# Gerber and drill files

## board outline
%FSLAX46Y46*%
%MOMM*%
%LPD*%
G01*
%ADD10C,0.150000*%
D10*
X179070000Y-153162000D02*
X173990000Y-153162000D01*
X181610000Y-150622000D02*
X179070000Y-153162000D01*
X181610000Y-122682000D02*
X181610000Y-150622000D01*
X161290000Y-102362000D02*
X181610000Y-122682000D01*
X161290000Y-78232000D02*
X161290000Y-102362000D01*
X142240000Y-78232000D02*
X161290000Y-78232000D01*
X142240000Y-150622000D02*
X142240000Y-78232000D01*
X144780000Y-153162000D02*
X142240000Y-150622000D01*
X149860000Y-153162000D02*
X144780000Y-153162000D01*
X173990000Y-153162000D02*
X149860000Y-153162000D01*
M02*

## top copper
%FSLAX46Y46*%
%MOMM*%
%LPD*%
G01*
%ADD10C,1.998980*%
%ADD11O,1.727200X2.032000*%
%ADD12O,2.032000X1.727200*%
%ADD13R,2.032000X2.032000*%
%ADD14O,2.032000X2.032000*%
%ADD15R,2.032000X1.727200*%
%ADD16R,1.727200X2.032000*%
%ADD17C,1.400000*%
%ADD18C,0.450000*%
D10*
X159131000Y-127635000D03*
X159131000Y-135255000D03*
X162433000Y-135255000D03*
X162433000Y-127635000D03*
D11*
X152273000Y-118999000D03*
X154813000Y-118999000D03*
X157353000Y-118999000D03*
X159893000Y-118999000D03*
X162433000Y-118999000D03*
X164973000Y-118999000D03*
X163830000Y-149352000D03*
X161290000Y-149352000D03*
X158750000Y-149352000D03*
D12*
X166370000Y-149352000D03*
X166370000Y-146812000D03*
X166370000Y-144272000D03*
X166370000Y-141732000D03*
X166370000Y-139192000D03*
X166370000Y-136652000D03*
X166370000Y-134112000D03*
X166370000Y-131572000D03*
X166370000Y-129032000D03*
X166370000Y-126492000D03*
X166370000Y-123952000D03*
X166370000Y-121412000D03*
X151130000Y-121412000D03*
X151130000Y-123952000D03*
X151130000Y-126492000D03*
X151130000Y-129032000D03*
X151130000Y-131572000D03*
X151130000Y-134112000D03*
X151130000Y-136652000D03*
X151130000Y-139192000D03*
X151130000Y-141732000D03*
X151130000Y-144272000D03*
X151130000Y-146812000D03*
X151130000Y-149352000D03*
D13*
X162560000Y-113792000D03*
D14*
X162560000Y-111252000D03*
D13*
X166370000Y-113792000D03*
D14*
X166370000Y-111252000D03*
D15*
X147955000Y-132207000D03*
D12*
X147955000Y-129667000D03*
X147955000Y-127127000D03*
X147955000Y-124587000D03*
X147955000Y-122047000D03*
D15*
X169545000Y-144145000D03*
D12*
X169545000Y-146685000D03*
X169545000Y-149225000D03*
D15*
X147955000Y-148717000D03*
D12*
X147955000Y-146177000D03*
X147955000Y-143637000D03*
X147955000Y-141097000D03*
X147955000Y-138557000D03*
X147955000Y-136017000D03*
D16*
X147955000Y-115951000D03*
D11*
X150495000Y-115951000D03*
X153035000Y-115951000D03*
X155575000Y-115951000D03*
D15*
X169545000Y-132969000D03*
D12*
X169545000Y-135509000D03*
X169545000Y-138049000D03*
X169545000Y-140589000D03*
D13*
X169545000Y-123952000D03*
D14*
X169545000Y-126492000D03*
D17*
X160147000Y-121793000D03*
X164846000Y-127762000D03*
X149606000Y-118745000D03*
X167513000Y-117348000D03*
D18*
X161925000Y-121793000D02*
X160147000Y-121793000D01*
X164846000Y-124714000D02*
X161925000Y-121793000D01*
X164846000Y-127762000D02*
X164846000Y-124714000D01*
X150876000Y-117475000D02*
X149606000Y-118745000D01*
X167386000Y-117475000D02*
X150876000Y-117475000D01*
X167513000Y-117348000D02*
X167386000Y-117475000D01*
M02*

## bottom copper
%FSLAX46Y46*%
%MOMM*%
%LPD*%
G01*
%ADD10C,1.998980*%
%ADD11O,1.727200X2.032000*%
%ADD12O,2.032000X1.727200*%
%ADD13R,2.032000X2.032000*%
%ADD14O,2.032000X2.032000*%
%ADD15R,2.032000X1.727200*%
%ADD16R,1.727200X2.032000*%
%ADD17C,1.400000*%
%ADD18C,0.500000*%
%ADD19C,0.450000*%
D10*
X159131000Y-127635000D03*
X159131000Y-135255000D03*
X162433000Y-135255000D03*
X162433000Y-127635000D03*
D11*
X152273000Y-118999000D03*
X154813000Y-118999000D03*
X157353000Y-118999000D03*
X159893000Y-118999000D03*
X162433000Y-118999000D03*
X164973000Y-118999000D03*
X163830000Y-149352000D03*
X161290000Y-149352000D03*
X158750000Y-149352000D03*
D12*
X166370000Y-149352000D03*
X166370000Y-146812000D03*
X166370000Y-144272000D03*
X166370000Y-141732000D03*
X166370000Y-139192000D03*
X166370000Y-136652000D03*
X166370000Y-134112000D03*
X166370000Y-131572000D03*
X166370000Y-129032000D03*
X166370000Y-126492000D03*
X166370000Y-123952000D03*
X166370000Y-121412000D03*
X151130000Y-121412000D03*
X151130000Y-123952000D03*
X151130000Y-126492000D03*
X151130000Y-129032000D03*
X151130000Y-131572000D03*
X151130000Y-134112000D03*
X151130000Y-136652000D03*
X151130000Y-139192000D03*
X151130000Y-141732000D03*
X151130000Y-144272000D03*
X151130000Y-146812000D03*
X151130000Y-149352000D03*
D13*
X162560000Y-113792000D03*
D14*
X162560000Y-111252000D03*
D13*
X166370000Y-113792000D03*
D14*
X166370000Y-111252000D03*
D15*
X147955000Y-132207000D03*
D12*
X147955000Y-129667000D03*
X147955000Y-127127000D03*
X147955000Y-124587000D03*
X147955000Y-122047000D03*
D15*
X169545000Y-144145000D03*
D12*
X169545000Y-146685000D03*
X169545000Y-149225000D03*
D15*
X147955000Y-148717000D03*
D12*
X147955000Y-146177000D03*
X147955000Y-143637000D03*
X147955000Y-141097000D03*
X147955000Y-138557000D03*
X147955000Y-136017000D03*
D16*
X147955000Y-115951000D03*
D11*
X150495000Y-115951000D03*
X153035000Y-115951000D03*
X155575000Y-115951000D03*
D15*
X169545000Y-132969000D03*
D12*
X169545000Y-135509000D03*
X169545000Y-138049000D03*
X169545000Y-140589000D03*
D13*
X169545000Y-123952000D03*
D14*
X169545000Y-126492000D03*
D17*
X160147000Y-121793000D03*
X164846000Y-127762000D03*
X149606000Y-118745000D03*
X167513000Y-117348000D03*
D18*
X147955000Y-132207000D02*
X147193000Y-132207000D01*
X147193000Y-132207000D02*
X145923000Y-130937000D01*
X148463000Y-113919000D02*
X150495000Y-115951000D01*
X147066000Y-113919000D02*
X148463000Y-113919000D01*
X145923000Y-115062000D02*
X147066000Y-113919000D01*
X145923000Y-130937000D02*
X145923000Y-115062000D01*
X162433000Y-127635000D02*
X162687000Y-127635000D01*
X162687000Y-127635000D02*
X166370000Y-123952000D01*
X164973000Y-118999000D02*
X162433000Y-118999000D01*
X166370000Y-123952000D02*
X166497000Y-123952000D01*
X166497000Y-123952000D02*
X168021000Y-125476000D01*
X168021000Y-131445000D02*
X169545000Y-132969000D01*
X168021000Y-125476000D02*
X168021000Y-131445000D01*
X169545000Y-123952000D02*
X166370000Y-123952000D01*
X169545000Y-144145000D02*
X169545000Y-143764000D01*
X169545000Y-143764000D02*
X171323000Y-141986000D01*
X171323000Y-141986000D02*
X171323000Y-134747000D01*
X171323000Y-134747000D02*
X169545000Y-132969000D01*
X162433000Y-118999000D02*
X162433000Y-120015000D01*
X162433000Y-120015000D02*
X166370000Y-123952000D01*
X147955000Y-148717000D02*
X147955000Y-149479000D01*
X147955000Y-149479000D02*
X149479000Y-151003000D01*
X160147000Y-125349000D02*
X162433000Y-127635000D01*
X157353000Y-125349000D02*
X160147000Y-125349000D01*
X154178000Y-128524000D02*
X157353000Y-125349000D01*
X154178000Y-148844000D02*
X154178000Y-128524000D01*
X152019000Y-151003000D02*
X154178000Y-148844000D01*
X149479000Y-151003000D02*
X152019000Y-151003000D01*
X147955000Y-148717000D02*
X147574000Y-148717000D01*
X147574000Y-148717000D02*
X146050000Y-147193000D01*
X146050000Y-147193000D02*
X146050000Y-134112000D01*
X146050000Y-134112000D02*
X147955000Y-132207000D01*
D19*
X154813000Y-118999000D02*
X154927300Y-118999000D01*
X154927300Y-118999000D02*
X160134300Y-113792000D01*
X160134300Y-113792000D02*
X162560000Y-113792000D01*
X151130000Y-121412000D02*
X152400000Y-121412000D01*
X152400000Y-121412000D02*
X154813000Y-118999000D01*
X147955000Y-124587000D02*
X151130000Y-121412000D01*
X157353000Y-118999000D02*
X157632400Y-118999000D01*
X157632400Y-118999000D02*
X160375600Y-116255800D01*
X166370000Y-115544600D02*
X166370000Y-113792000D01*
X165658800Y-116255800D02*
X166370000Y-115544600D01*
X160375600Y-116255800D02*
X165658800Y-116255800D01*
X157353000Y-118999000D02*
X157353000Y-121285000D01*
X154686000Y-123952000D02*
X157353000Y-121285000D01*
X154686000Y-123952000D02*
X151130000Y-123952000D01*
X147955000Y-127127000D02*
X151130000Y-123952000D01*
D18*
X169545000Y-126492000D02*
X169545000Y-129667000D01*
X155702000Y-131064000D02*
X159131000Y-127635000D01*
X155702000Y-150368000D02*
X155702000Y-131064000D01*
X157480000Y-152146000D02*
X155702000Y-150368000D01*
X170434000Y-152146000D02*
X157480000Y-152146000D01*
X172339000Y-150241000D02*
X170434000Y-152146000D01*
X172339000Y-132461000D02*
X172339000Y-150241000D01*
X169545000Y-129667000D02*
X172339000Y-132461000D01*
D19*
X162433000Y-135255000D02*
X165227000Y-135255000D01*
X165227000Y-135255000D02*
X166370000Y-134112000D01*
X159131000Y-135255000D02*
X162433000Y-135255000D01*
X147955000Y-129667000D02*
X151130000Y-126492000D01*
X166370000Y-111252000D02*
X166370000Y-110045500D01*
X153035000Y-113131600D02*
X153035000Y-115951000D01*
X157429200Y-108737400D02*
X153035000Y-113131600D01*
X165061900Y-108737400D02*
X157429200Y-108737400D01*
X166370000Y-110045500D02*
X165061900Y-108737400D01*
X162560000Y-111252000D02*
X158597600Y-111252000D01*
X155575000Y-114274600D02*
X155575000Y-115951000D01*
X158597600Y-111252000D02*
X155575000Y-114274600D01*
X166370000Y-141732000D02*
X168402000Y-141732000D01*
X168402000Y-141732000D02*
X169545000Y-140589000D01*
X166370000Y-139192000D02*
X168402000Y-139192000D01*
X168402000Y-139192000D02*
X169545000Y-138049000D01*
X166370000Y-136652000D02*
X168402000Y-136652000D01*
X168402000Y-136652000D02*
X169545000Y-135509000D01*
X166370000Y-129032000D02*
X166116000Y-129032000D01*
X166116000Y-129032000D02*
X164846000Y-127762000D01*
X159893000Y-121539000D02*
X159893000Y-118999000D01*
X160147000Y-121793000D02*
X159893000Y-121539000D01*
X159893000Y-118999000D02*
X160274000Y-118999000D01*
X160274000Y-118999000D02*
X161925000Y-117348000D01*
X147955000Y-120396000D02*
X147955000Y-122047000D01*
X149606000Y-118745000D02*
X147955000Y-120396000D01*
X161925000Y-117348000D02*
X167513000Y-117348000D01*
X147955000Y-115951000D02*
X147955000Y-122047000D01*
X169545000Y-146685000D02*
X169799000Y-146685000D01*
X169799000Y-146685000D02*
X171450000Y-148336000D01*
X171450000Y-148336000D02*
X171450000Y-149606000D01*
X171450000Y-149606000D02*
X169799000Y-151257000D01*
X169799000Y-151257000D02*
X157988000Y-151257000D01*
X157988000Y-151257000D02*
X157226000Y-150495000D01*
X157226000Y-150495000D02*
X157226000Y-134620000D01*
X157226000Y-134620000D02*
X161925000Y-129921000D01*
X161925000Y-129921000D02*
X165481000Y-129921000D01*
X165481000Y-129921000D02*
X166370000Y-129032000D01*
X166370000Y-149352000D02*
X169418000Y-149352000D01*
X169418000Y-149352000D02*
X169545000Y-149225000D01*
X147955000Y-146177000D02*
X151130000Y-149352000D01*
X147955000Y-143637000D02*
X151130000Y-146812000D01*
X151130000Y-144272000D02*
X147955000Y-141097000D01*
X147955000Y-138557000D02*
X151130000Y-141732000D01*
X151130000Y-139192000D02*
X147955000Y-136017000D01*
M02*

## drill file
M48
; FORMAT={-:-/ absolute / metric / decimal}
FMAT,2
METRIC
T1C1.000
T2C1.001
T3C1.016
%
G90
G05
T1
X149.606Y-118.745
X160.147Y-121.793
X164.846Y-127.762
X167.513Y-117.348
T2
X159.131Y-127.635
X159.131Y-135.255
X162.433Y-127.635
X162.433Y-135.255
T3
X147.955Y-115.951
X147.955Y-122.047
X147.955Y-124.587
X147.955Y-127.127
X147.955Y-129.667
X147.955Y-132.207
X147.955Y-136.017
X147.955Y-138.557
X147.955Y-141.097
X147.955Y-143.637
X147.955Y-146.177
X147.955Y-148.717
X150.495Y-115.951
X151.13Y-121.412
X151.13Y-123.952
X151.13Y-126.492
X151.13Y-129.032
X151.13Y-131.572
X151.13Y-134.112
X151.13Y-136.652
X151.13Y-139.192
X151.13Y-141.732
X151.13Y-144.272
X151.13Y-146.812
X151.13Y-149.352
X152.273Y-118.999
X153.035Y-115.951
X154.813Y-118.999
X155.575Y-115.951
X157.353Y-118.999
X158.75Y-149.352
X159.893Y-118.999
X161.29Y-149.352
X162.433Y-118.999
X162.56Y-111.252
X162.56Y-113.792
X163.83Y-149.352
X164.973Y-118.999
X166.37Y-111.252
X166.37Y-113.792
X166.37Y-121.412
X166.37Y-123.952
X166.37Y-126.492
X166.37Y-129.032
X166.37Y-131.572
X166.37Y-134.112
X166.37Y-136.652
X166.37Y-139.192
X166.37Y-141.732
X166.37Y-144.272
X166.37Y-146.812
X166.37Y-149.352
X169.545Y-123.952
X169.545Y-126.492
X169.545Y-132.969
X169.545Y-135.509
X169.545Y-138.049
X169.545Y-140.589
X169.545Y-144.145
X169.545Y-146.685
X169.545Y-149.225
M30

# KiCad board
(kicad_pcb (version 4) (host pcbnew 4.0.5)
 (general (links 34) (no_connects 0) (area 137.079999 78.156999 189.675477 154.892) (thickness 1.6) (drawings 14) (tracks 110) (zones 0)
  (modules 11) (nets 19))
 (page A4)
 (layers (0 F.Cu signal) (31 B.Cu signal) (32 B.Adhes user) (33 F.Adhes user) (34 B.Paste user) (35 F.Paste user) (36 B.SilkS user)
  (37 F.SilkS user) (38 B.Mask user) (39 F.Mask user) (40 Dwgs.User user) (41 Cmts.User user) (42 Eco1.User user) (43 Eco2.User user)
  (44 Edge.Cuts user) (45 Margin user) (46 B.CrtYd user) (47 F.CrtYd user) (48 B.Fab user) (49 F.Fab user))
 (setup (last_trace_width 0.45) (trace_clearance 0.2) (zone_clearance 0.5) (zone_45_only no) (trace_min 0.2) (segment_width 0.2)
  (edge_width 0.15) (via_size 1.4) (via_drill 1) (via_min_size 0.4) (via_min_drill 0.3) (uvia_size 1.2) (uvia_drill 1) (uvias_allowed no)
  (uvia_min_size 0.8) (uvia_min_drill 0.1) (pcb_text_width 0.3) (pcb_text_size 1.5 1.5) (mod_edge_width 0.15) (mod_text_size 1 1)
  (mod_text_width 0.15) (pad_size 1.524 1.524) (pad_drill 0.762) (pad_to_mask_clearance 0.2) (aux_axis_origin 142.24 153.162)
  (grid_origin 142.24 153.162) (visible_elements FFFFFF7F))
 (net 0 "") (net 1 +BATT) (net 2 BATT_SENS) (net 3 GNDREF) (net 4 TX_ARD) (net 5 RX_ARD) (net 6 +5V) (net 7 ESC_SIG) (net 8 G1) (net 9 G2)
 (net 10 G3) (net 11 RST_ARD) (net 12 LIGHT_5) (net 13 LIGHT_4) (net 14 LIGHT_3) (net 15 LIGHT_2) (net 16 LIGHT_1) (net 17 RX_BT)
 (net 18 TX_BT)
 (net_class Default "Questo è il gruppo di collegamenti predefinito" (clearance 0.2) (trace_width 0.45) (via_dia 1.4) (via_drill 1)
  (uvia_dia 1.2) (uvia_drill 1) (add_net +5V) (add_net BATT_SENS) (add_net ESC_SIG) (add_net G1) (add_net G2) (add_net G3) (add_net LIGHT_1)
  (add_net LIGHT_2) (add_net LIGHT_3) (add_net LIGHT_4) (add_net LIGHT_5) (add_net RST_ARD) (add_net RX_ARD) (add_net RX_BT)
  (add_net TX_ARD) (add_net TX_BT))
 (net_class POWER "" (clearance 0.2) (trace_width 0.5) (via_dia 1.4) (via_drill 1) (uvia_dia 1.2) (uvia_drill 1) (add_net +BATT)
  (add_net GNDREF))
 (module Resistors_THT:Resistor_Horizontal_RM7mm (layer F.Cu) (at 159.131 127.635 270)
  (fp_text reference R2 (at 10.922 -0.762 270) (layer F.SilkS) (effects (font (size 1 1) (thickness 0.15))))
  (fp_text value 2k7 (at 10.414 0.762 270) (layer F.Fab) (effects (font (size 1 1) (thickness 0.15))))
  (pad 1 thru_hole circle (at 0 0 270) (size 1.99898 1.99898) (drill 1.00076) (layers *.Cu *.SilkS *.Mask) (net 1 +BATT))
  (pad 2 thru_hole circle (at 7.62 0 270) (size 1.99898 1.99898) (drill 1.00076) (layers *.Cu *.SilkS *.Mask) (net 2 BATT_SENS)))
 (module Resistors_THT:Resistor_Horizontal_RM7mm (layer F.Cu) (at 162.433 135.255 90)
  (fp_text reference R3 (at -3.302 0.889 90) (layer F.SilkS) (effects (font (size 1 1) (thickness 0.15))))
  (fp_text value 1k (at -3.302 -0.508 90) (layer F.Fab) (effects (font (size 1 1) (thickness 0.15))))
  (pad 1 thru_hole circle (at 0 0 90) (size 1.99898 1.99898) (drill 1.00076) (layers *.Cu *.SilkS *.Mask) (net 2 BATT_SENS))
  (pad 2 thru_hole circle (at 7.62 0 90) (size 1.99898 1.99898) (drill 1.00076) (layers *.Cu *.SilkS *.Mask) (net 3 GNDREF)))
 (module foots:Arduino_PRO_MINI (layer F.Cu) (at 158.75 118.872)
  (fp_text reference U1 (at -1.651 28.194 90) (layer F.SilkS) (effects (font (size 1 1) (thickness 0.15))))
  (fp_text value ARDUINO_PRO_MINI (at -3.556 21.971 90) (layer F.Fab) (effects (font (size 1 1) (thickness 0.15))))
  (pad 33 thru_hole oval (at -6.477 0.127 90) (size 2.032 1.7272) (drill 1.016) (layers *.Cu *.Mask))
  (pad 32 thru_hole oval (at -3.937 0.127 90) (size 2.032 1.7272) (drill 1.016) (layers *.Cu *.Mask) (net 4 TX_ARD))
  (pad 31 thru_hole oval (at -1.397 0.127 90) (size 2.032 1.7272) (drill 1.016) (layers *.Cu *.Mask) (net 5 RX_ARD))
  (pad 30 thru_hole oval (at 1.143 0.127 90) (size 2.032 1.7272) (drill 1.016) (layers *.Cu *.Mask) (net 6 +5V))
  (pad 29 thru_hole oval (at 3.683 0.127 90) (size 2.032 1.7272) (drill 1.016) (layers *.Cu *.Mask) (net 3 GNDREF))
  (pad 28 thru_hole oval (at 6.223 0.127 90) (size 2.032 1.7272) (drill 1.016) (layers *.Cu *.Mask) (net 3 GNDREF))
  (pad 15 thru_hole oval (at 5.08 30.48 90) (size 2.032 1.7272) (drill 1.016) (layers *.Cu *.Mask))
  (pad 14 thru_hole oval (at 2.54 30.48 90) (size 2.032 1.7272) (drill 1.016) (layers *.Cu *.Mask))
  (pad 13 thru_hole oval (at 0 30.48 90) (size 2.032 1.7272) (drill 1.016) (layers *.Cu *.Mask))
  (pad 16 thru_hole oval (at 7.62 30.48) (size 2.032 1.7272) (drill 1.016) (layers *.Cu *.Mask) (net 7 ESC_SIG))
  (pad 17 thru_hole oval (at 7.62 27.94) (size 2.032 1.7272) (drill 1.016) (layers *.Cu *.Mask))
  (pad 18 thru_hole oval (at 7.62 25.4) (size 2.032 1.7272) (drill 1.016) (layers *.Cu *.Mask))
  (pad 19 thru_hole oval (at 7.62 22.86) (size 2.032 1.7272) (drill 1.016) (layers *.Cu *.Mask) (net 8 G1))
  (pad 20 thru_hole oval (at 7.62 20.32) (size 2.032 1.7272) (drill 1.016) (layers *.Cu *.Mask) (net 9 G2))
  (pad 21 thru_hole oval (at 7.62 17.78) (size 2.032 1.7272) (drill 1.016) (layers *.Cu *.Mask) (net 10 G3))
  (pad 22 thru_hole oval (at 7.62 15.24) (size 2.032 1.7272) (drill 1.016) (layers *.Cu *.Mask) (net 2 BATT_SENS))
  (pad 23 thru_hole oval (at 7.62 12.7) (size 2.032 1.7272) (drill 1.016) (layers *.Cu *.Mask))
  (pad 24 thru_hole oval (at 7.62 10.16) (size 2.032 1.7272) (drill 1.016) (layers *.Cu *.Mask) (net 6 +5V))
  (pad 25 thru_hole oval (at 7.62 7.62) (size 2.032 1.7272) (drill 1.016) (layers *.Cu *.Mask))
  (pad 26 thru_hole oval (at 7.62 5.08) (size 2.032 1.7272) (drill 1.016) (layers *.Cu *.Mask) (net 3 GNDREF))
  (pad 27 thru_hole oval (at 7.62 2.54) (size 2.032 1.7272) (drill 1.016) (layers *.Cu *.Mask))
  (pad 1 thru_hole oval (at -7.62 2.54) (size 2.032 1.7272) (drill 1.016) (layers *.Cu *.Mask) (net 4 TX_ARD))
  (pad 2 thru_hole oval (at -7.62 5.08) (size 2.032 1.7272) (drill 1.016) (layers *.Cu *.Mask) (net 5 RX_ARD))
  (pad 3 thru_hole oval (at -7.62 7.62) (size 2.032 1.7272) (drill 1.016) (layers *.Cu *.Mask) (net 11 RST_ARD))
  (pad 4 thru_hole oval (at -7.62 10.16) (size 2.032 1.7272) (drill 1.016) (layers *.Cu *.Mask))
  (pad 5 thru_hole oval (at -7.62 12.7) (size 2.032 1.7272) (drill 1.016) (layers *.Cu *.Mask))
  (pad 6 thru_hole oval (at -7.62 15.24) (size 2.032 1.7272) (drill 1.016) (layers *.Cu *.Mask))
  (pad 7 thru_hole oval (at -7.62 17.78) (size 2.032 1.7272) (drill 1.016) (layers *.Cu *.Mask))
  (pad 8 thru_hole oval (at -7.62 20.32) (size 2.032 1.7272) (drill 1.016) (layers *.Cu *.Mask) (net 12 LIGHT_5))
  (pad 9 thru_hole oval (at -7.62 22.86) (size 2.032 1.7272) (drill 1.016) (layers *.Cu *.Mask) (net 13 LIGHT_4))
  (pad 10 thru_hole oval (at -7.62 25.4) (size 2.032 1.7272) (drill 1.016) (layers *.Cu *.Mask) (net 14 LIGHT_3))
  (pad 11 thru_hole oval (at -7.62 27.94) (size 2.032 1.7272) (drill 1.016) (layers *.Cu *.Mask) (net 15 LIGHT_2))
  (pad 12 thru_hole oval (at -7.62 30.48) (size 2.032 1.7272) (drill 1.016) (layers *.Cu *.Mask) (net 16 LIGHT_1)))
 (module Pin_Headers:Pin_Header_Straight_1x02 (layer F.Cu) (at 162.56 113.792 180)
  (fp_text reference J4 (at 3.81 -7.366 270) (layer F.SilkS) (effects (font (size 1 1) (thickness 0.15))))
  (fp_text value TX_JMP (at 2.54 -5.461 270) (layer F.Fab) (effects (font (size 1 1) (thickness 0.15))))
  (pad 1 thru_hole rect (at 0 0 180) (size 2.032 2.032) (drill 1.016) (layers *.Cu *.Mask) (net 4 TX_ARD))
  (pad 2 thru_hole oval (at 0 2.54 180) (size 2.032 2.032) (drill 1.016) (layers *.Cu *.Mask) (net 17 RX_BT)))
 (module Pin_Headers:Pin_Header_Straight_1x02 (layer F.Cu) (at 166.37 113.792 180)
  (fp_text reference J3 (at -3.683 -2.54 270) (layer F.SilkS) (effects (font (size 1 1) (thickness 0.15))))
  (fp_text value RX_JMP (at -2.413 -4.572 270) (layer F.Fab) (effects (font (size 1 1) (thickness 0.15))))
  (pad 1 thru_hole rect (at 0 0 180) (size 2.032 2.032) (drill 1.016) (layers *.Cu *.Mask) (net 5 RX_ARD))
  (pad 2 thru_hole oval (at 0 2.54 180) (size 2.032 2.032) (drill 1.016) (layers *.Cu *.Mask) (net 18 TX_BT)))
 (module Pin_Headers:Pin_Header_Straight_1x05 (layer F.Cu) (at 147.955 132.207 180)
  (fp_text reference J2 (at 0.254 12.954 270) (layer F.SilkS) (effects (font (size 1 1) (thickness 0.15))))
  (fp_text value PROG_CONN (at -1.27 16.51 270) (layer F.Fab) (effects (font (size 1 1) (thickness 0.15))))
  (pad 1 thru_hole rect (at 0 0 180) (size 2.032 1.7272) (drill 1.016) (layers *.Cu *.Mask) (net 3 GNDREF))
  (pad 2 thru_hole oval (at 0 2.54 180) (size 2.032 1.7272) (drill 1.016) (layers *.Cu *.Mask) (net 11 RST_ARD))
  (pad 3 thru_hole oval (at 0 5.08 180) (size 2.032 1.7272) (drill 1.016) (layers *.Cu *.Mask) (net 5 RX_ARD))
  (pad 4 thru_hole oval (at 0 7.62 180) (size 2.032 1.7272) (drill 1.016) (layers *.Cu *.Mask) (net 4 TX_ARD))
  (pad 5 thru_hole oval (at 0 10.16 180) (size 2.032 1.7272) (drill 1.016) (layers *.Cu *.Mask) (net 6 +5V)))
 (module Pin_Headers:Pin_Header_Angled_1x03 (layer F.Cu) (at 169.545 144.145)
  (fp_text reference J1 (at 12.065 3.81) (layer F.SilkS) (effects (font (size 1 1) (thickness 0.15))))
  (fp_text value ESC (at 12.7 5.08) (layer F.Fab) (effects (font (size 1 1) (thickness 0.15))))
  (pad 1 thru_hole rect (at 0 0) (size 2.032 1.7272) (drill 1.016) (layers *.Cu *.Mask) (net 3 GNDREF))
  (pad 2 thru_hole oval (at 0 2.54) (size 2.032 1.7272) (drill 1.016) (layers *.Cu *.Mask) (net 6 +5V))
  (pad 3 thru_hole oval (at 0 5.08) (size 2.032 1.7272) (drill 1.016) (layers *.Cu *.Mask) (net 7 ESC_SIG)))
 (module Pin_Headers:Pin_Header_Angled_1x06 (layer F.Cu) (at 147.955 148.717 180)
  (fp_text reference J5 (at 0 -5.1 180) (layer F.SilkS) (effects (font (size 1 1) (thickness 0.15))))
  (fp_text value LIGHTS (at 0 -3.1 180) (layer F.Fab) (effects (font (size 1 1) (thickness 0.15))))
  (pad 1 thru_hole rect (at 0 0 180) (size 2.032 1.7272) (drill 1.016) (layers *.Cu *.Mask) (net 3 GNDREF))
  (pad 2 thru_hole oval (at 0 2.54 180) (size 2.032 1.7272) (drill 1.016) (layers *.Cu *.Mask) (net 16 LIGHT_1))
  (pad 3 thru_hole oval (at 0 5.08 180) (size 2.032 1.7272) (drill 1.016) (layers *.Cu *.Mask) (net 15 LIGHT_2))
  (pad 4 thru_hole oval (at 0 7.62 180) (size 2.032 1.7272) (drill 1.016) (layers *.Cu *.Mask) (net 14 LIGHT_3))
  (pad 5 thru_hole oval (at 0 10.16 180) (size 2.032 1.7272) (drill 1.016) (layers *.Cu *.Mask) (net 13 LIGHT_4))
  (pad 6 thru_hole oval (at 0 12.7 180) (size 2.032 1.7272) (drill 1.016) (layers *.Cu *.Mask) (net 12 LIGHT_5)))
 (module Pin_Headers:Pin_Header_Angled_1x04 (layer F.Cu) (at 147.955 115.951 90)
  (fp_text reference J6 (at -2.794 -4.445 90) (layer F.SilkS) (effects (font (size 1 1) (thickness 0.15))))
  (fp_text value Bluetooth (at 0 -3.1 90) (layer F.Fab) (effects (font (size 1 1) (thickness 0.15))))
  (pad 1 thru_hole rect (at 0 0 90) (size 2.032 1.7272) (drill 1.016) (layers *.Cu *.Mask) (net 6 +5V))
  (pad 2 thru_hole oval (at 0 2.54 90) (size 2.032 1.7272) (drill 1.016) (layers *.Cu *.Mask) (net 3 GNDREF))
  (pad 3 thru_hole oval (at 0 5.08 90) (size 2.032 1.7272) (drill 1.016) (layers *.Cu *.Mask) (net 18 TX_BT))
  (pad 4 thru_hole oval (at 0 7.62 90) (size 2.032 1.7272) (drill 1.016) (layers *.Cu *.Mask) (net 17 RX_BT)))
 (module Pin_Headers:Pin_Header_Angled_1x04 (layer F.Cu) (at 169.545 132.969)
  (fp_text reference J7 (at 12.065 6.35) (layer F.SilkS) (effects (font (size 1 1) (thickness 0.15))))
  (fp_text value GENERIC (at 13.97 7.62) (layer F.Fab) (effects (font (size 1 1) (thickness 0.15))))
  (pad 1 thru_hole rect (at 0 0) (size 2.032 1.7272) (drill 1.016) (layers *.Cu *.Mask) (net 3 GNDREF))
  (pad 2 thru_hole oval (at 0 2.54) (size 2.032 1.7272) (drill 1.016) (layers *.Cu *.Mask) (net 10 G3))
  (pad 3 thru_hole oval (at 0 5.08) (size 2.032 1.7272) (drill 1.016) (layers *.Cu *.Mask) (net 9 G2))
  (pad 4 thru_hole oval (at 0 7.62) (size 2.032 1.7272) (drill 1.016) (layers *.Cu *.Mask) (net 8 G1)))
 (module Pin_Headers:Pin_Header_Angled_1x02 (layer F.Cu) (at 169.545 123.952)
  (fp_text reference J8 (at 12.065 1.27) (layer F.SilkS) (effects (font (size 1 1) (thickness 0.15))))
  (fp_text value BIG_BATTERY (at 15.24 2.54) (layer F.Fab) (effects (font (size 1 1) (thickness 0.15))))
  (pad 1 thru_hole rect (at 0 0) (size 2.032 2.032) (drill 1.016) (layers *.Cu *.Mask) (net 3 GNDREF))
  (pad 2 thru_hole oval (at 0 2.54) (size 2.032 2.032) (drill 1.016) (layers *.Cu *.Mask) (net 1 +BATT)))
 (gr_line (start 179.07 153.162) (end 173.99 153.162) (angle 90) (layer Edge.Cuts) (width 0.15))
 (gr_line (start 181.61 150.622) (end 179.07 153.162) (angle 90) (layer Edge.Cuts) (width 0.15))
 (gr_line (start 181.61 122.682) (end 181.61 150.622) (angle 90) (layer Edge.Cuts) (width 0.15))
 (gr_line (start 161.29 102.362) (end 181.61 122.682) (angle 90) (layer Edge.Cuts) (width 0.15))
 (gr_line (start 161.29 78.232) (end 161.29 102.362) (angle 90) (layer Edge.Cuts) (width 0.15))
 (gr_line (start 142.24 78.232) (end 161.29 78.232) (angle 90) (layer Edge.Cuts) (width 0.15))
 (gr_line (start 142.24 150.622) (end 142.24 78.232) (angle 90) (layer Edge.Cuts) (width 0.15))
 (gr_line (start 144.78 153.162) (end 142.24 150.622) (angle 90) (layer Edge.Cuts) (width 0.15))
 (gr_line (start 149.86 153.162) (end 144.78 153.162) (angle 90) (layer Edge.Cuts) (width 0.15))
 (gr_line (start 173.99 153.162) (end 149.86 153.162) (angle 90) (layer Edge.Cuts) (width 0.15))
 (segment (start 147.955 132.207) (end 147.193 132.207) (width 0.5) (layer B.Cu) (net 3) (status 30))
 (segment (start 147.193 132.207) (end 145.923 130.937) (width 0.5) (layer B.Cu) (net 3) (status 10))
 (segment (start 148.463 113.919) (end 150.495 115.951) (width 0.5) (layer B.Cu) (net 3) (status 20))
 (segment (start 147.066 113.919) (end 148.463 113.919) (width 0.5) (layer B.Cu) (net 3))
 (segment (start 145.923 115.062) (end 147.066 113.919) (width 0.5) (layer B.Cu) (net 3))
 (segment (start 145.923 130.937) (end 145.923 115.062) (width 0.5) (layer B.Cu) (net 3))
 (segment (start 162.433 127.635) (end 162.687 127.635) (width 0.5) (layer B.Cu) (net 3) (status 30))
 (segment (start 162.687 127.635) (end 166.37 123.952) (width 0.5) (layer B.Cu) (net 3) (status 30))
 (segment (start 164.973 118.999) (end 162.433 118.999) (width 0.5) (layer B.Cu) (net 3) (status 30))
 (segment (start 166.37 123.952) (end 166.497 123.952) (width 0.5) (layer B.Cu) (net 3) (status 30))
 (segment (start 166.497 123.952) (end 168.021 125.476) (width 0.5) (layer B.Cu) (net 3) (status 10))
 (segment (start 168.021 131.445) (end 169.545 132.969) (width 0.5) (layer B.Cu) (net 3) (status 20))
 (segment (start 168.021 125.476) (end 168.021 131.445) (width 0.5) (layer B.Cu) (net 3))
 (segment (start 169.545 123.952) (end 166.37 123.952) (width 0.5) (layer B.Cu) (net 3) (status 30))
 (segment (start 169.545 144.145) (end 169.545 143.764) (width 0.5) (layer B.Cu) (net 3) (status 30))
 (segment (start 169.545 143.764) (end 171.323 141.986) (width 0.5) (layer B.Cu) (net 3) (status 10))
 (segment (start 171.323 141.986) (end 171.323 134.747) (width 0.5) (layer B.Cu) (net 3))
 (segment (start 171.323 134.747) (end 169.545 132.969) (width 0.5) (layer B.Cu) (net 3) (status 20))
 (segment (start 162.433 118.999) (end 162.433 120.015) (width 0.5) (layer B.Cu) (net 3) (status 30))
 (segment (start 162.433 120.015) (end 166.37 123.952) (width 0.5) (layer B.Cu) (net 3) (status 30))
 (segment (start 147.955 148.717) (end 147.955 149.479) (width 0.5) (layer B.Cu) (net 3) (status 30))
 (segment (start 147.955 149.479) (end 149.479 151.003) (width 0.5) (layer B.Cu) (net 3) (status 10))
 (segment (start 160.147 125.349) (end 162.433 127.635) (width 0.5) (layer B.Cu) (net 3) (status 20))
 (segment (start 157.353 125.349) (end 160.147 125.349) (width 0.5) (layer B.Cu) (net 3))
 (segment (start 154.178 128.524) (end 157.353 125.349) (width 0.5) (layer B.Cu) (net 3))
 (segment (start 154.178 148.844) (end 154.178 128.524) (width 0.5) (layer B.Cu) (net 3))
 (segment (start 152.019 151.003) (end 154.178 148.844) (width 0.5) (layer B.Cu) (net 3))
 (segment (start 149.479 151.003) (end 152.019 151.003) (width 0.5) (layer B.Cu) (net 3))
 (segment (start 147.955 148.717) (end 147.574 148.717) (width 0.5) (layer B.Cu) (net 3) (status 30))
 (segment (start 147.574 148.717) (end 146.05 147.193) (width 0.5) (layer B.Cu) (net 3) (status 10))
 (segment (start 146.05 147.193) (end 146.05 134.112) (width 0.5) (layer B.Cu) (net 3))
 (segment (start 146.05 134.112) (end 147.955 132.207) (width 0.5) (layer B.Cu) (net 3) (status 20))
 (segment (start 154.813 118.999) (end 154.9273 118.999) (width 0.45) (layer B.Cu) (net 4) (status C00000))
 (segment (start 154.9273 118.999) (end 160.1343 113.792) (width 0.45) (layer B.Cu) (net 4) (status 400000))
 (segment (start 160.1343 113.792) (end 162.56 113.792) (width 0.45) (layer B.Cu) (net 4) (status 800000))
 (segment (start 151.13 121.412) (end 152.4 121.412) (width 0.45) (layer B.Cu) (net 4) (status 10))
 (segment (start 152.4 121.412) (end 154.813 118.999) (width 0.45) (layer B.Cu) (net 4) (status 20))
 (segment (start 147.955 124.587) (end 151.13 121.412) (width 0.45) (layer B.Cu) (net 4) (status 30))
 (segment (start 157.353 118.999) (end 157.6324 118.999) (width 0.45) (layer B.Cu) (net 5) (status C00000))
 (segment (start 157.6324 118.999) (end 160.3756 116.2558) (width 0.45) (layer B.Cu) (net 5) (status 400000))
 (segment (start 166.37 115.5446) (end 166.37 113.792) (width 0.45) (layer B.Cu) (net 5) (status 800000))
 (segment (start 165.6588 116.2558) (end 166.37 115.5446) (width 0.45) (layer B.Cu) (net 5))
 (segment (start 160.3756 116.2558) (end 165.6588 116.2558) (width 0.45) (layer B.Cu) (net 5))
 (segment (start 157.353 118.999) (end 157.353 121.285) (width 0.45) (layer B.Cu) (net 5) (status 10))
 (segment (start 154.686 123.952) (end 157.353 121.285) (width 0.45) (layer B.Cu) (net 5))
 (segment (start 154.686 123.952) (end 151.13 123.952) (width 0.45) (layer B.Cu) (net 5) (status 20))
 (segment (start 147.955 127.127) (end 151.13 123.952) (width 0.45) (layer B.Cu) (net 5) (status 30))
 (segment (start 169.545 126.492) (end 169.545 129.667) (width 0.5) (layer B.Cu) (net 1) (status 10))
 (segment (start 155.702 131.064) (end 159.131 127.635) (width 0.5) (layer B.Cu) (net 1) (status 20))
 (segment (start 155.702 150.368) (end 155.702 131.064) (width 0.5) (layer B.Cu) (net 1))
 (segment (start 157.48 152.146) (end 155.702 150.368) (width 0.5) (layer B.Cu) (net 1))
 (segment (start 170.434 152.146) (end 157.48 152.146) (width 0.5) (layer B.Cu) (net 1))
 (segment (start 172.339 150.241) (end 170.434 152.146) (width 0.5) (layer B.Cu) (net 1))
 (segment (start 172.339 132.461) (end 172.339 150.241) (width 0.5) (layer B.Cu) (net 1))
 (segment (start 169.545 129.667) (end 172.339 132.461) (width 0.5) (layer B.Cu) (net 1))
 (segment (start 162.433 135.255) (end 165.227 135.255) (width 0.45) (layer B.Cu) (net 2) (status 10))
 (segment (start 165.227 135.255) (end 166.37 134.112) (width 0.45) (layer B.Cu) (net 2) (status 20))
 (segment (start 159.131 135.255) (end 162.433 135.255) (width 0.45) (layer B.Cu) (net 2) (status 30))
 (segment (start 147.955 129.667) (end 151.13 126.492) (width 0.45) (layer B.Cu) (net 11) (status 30))
 (segment (start 166.37 111.252) (end 166.37 110.0455) (width 0.45) (layer B.Cu) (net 18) (status 400000))
 (segment (start 153.035 113.1316) (end 153.035 115.951) (width 0.45) (layer B.Cu) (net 18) (status 800000))
 (segment (start 157.4292 108.7374) (end 153.035 113.1316) (width 0.45) (layer B.Cu) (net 18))
 (segment (start 165.0619 108.7374) (end 157.4292 108.7374) (width 0.45) (layer B.Cu) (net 18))
 (segment (start 166.37 110.0455) (end 165.0619 108.7374) (width 0.45) (layer B.Cu) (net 18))
 (segment (start 162.56 111.252) (end 158.5976 111.252) (width 0.45) (layer B.Cu) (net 17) (status 400000))
 (segment (start 155.575 114.2746) (end 155.575 115.951) (width 0.45) (layer B.Cu) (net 17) (status 800000))
 (segment (start 158.5976 111.252) (end 155.575 114.2746) (width 0.45) (layer B.Cu) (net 17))
 (segment (start 166.37 141.732) (end 168.402 141.732) (width 0.45) (layer B.Cu) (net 8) (status 10))
 (segment (start 168.402 141.732) (end 169.545 140.589) (width 0.45) (layer B.Cu) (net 8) (status 20))
 (segment (start 166.37 139.192) (end 168.402 139.192) (width 0.45) (layer B.Cu) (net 9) (status 10))
 (segment (start 168.402 139.192) (end 169.545 138.049) (width 0.45) (layer B.Cu) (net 9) (status 20))
 (segment (start 166.37 136.652) (end 168.402 136.652) (width 0.45) (layer B.Cu) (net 10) (status 10))
 (segment (start 168.402 136.652) (end 169.545 135.509) (width 0.45) (layer B.Cu) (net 10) (status 20))
 (segment (start 166.37 129.032) (end 166.116 129.032) (width 0.45) (layer B.Cu) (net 6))
 (segment (start 166.116 129.032) (end 164.846 127.762) (width 0.45) (layer B.Cu) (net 6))
 (segment (start 159.893 121.539) (end 159.893 118.999) (width 0.45) (layer B.Cu) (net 6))
 (segment (start 160.147 121.793) (end 159.893 121.539) (width 0.45) (layer B.Cu) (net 6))
 (via (at 160.147 121.793) (size 1.4) (drill 1) (layers F.Cu B.Cu) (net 6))
 (segment (start 161.925 121.793) (end 160.147 121.793) (width 0.45) (layer F.Cu) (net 6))
 (segment (start 164.846 124.714) (end 161.925 121.793) (width 0.45) (layer F.Cu) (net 6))
 (segment (start 164.846 127.762) (end 164.846 124.714) (width 0.45) (layer F.Cu) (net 6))
 (via (at 164.846 127.762) (size 1.4) (drill 1) (layers F.Cu B.Cu) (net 6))
 (segment (start 159.893 118.999) (end 160.274 118.999) (width 0.45) (layer B.Cu) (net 6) (status 30))
 (segment (start 160.274 118.999) (end 161.925 117.348) (width 0.45) (layer B.Cu) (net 6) (status 10))
 (segment (start 147.955 120.396) (end 147.955 122.047) (width 0.45) (layer B.Cu) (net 6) (status 20))
 (segment (start 149.606 118.745) (end 147.955 120.396) (width 0.45) (layer B.Cu) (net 6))
 (via (at 149.606 118.745) (size 1.4) (drill 1) (layers F.Cu B.Cu) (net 6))
 (segment (start 150.876 117.475) (end 149.606 118.745) (width 0.45) (layer F.Cu) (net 6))
 (segment (start 167.386 117.475) (end 150.876 117.475) (width 0.45) (layer F.Cu) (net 6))
 (segment (start 167.513 117.348) (end 167.386 117.475) (width 0.45) (layer F.Cu) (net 6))
 (via (at 167.513 117.348) (size 1.4) (drill 1) (layers F.Cu B.Cu) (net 6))
 (segment (start 161.925 117.348) (end 167.513 117.348) (width 0.45) (layer B.Cu) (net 6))
 (segment (start 147.955 115.951) (end 147.955 122.047) (width 0.45) (layer B.Cu) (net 6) (status 30))
 (segment (start 169.545 146.685) (end 169.799 146.685) (width 0.45) (layer B.Cu) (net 6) (status 30))
 (segment (start 169.799 146.685) (end 171.45 148.336) (width 0.45) (layer B.Cu) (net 6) (status 10))
 (segment (start 171.45 148.336) (end 171.45 149.606) (width 0.45) (layer B.Cu) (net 6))
 (segment (start 171.45 149.606) (end 169.799 151.257) (width 0.45) (layer B.Cu) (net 6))
 (segment (start 169.799 151.257) (end 157.988 151.257) (width 0.45) (layer B.Cu) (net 6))
 (segment (start 157.988 151.257) (end 157.226 150.495) (width 0.45) (layer B.Cu) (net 6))
 (segment (start 157.226 150.495) (end 157.226 134.62) (width 0.45) (layer B.Cu) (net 6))
 (segment (start 157.226 134.62) (end 161.925 129.921) (width 0.45) (layer B.Cu) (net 6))
 (segment (start 161.925 129.921) (end 165.481 129.921) (width 0.45) (layer B.Cu) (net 6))
 (segment (start 165.481 129.921) (end 166.37 129.032) (width 0.45) (layer B.Cu) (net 6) (status 20))
 (segment (start 166.37 149.352) (end 169.418 149.352) (width 0.45) (layer B.Cu) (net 7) (status 30))
 (segment (start 169.418 149.352) (end 169.545 149.225) (width 0.45) (layer B.Cu) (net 7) (status 30))
 (segment (start 147.955 146.177) (end 151.13 149.352) (width 0.45) (layer B.Cu) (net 16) (status 30))
 (segment (start 147.955 143.637) (end 151.13 146.812) (width 0.45) (layer B.Cu) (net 15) (status 30))
 (segment (start 151.13 144.272) (end 147.955 141.097) (width 0.45) (layer B.Cu) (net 14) (status 30))
 (segment (start 147.955 138.557) (end 151.13 141.732) (width 0.45) (layer B.Cu) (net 13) (status 30))
 (segment (start 151.13 139.192) (end 147.955 136.017) (width 0.45) (layer B.Cu) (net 12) (status 30)))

